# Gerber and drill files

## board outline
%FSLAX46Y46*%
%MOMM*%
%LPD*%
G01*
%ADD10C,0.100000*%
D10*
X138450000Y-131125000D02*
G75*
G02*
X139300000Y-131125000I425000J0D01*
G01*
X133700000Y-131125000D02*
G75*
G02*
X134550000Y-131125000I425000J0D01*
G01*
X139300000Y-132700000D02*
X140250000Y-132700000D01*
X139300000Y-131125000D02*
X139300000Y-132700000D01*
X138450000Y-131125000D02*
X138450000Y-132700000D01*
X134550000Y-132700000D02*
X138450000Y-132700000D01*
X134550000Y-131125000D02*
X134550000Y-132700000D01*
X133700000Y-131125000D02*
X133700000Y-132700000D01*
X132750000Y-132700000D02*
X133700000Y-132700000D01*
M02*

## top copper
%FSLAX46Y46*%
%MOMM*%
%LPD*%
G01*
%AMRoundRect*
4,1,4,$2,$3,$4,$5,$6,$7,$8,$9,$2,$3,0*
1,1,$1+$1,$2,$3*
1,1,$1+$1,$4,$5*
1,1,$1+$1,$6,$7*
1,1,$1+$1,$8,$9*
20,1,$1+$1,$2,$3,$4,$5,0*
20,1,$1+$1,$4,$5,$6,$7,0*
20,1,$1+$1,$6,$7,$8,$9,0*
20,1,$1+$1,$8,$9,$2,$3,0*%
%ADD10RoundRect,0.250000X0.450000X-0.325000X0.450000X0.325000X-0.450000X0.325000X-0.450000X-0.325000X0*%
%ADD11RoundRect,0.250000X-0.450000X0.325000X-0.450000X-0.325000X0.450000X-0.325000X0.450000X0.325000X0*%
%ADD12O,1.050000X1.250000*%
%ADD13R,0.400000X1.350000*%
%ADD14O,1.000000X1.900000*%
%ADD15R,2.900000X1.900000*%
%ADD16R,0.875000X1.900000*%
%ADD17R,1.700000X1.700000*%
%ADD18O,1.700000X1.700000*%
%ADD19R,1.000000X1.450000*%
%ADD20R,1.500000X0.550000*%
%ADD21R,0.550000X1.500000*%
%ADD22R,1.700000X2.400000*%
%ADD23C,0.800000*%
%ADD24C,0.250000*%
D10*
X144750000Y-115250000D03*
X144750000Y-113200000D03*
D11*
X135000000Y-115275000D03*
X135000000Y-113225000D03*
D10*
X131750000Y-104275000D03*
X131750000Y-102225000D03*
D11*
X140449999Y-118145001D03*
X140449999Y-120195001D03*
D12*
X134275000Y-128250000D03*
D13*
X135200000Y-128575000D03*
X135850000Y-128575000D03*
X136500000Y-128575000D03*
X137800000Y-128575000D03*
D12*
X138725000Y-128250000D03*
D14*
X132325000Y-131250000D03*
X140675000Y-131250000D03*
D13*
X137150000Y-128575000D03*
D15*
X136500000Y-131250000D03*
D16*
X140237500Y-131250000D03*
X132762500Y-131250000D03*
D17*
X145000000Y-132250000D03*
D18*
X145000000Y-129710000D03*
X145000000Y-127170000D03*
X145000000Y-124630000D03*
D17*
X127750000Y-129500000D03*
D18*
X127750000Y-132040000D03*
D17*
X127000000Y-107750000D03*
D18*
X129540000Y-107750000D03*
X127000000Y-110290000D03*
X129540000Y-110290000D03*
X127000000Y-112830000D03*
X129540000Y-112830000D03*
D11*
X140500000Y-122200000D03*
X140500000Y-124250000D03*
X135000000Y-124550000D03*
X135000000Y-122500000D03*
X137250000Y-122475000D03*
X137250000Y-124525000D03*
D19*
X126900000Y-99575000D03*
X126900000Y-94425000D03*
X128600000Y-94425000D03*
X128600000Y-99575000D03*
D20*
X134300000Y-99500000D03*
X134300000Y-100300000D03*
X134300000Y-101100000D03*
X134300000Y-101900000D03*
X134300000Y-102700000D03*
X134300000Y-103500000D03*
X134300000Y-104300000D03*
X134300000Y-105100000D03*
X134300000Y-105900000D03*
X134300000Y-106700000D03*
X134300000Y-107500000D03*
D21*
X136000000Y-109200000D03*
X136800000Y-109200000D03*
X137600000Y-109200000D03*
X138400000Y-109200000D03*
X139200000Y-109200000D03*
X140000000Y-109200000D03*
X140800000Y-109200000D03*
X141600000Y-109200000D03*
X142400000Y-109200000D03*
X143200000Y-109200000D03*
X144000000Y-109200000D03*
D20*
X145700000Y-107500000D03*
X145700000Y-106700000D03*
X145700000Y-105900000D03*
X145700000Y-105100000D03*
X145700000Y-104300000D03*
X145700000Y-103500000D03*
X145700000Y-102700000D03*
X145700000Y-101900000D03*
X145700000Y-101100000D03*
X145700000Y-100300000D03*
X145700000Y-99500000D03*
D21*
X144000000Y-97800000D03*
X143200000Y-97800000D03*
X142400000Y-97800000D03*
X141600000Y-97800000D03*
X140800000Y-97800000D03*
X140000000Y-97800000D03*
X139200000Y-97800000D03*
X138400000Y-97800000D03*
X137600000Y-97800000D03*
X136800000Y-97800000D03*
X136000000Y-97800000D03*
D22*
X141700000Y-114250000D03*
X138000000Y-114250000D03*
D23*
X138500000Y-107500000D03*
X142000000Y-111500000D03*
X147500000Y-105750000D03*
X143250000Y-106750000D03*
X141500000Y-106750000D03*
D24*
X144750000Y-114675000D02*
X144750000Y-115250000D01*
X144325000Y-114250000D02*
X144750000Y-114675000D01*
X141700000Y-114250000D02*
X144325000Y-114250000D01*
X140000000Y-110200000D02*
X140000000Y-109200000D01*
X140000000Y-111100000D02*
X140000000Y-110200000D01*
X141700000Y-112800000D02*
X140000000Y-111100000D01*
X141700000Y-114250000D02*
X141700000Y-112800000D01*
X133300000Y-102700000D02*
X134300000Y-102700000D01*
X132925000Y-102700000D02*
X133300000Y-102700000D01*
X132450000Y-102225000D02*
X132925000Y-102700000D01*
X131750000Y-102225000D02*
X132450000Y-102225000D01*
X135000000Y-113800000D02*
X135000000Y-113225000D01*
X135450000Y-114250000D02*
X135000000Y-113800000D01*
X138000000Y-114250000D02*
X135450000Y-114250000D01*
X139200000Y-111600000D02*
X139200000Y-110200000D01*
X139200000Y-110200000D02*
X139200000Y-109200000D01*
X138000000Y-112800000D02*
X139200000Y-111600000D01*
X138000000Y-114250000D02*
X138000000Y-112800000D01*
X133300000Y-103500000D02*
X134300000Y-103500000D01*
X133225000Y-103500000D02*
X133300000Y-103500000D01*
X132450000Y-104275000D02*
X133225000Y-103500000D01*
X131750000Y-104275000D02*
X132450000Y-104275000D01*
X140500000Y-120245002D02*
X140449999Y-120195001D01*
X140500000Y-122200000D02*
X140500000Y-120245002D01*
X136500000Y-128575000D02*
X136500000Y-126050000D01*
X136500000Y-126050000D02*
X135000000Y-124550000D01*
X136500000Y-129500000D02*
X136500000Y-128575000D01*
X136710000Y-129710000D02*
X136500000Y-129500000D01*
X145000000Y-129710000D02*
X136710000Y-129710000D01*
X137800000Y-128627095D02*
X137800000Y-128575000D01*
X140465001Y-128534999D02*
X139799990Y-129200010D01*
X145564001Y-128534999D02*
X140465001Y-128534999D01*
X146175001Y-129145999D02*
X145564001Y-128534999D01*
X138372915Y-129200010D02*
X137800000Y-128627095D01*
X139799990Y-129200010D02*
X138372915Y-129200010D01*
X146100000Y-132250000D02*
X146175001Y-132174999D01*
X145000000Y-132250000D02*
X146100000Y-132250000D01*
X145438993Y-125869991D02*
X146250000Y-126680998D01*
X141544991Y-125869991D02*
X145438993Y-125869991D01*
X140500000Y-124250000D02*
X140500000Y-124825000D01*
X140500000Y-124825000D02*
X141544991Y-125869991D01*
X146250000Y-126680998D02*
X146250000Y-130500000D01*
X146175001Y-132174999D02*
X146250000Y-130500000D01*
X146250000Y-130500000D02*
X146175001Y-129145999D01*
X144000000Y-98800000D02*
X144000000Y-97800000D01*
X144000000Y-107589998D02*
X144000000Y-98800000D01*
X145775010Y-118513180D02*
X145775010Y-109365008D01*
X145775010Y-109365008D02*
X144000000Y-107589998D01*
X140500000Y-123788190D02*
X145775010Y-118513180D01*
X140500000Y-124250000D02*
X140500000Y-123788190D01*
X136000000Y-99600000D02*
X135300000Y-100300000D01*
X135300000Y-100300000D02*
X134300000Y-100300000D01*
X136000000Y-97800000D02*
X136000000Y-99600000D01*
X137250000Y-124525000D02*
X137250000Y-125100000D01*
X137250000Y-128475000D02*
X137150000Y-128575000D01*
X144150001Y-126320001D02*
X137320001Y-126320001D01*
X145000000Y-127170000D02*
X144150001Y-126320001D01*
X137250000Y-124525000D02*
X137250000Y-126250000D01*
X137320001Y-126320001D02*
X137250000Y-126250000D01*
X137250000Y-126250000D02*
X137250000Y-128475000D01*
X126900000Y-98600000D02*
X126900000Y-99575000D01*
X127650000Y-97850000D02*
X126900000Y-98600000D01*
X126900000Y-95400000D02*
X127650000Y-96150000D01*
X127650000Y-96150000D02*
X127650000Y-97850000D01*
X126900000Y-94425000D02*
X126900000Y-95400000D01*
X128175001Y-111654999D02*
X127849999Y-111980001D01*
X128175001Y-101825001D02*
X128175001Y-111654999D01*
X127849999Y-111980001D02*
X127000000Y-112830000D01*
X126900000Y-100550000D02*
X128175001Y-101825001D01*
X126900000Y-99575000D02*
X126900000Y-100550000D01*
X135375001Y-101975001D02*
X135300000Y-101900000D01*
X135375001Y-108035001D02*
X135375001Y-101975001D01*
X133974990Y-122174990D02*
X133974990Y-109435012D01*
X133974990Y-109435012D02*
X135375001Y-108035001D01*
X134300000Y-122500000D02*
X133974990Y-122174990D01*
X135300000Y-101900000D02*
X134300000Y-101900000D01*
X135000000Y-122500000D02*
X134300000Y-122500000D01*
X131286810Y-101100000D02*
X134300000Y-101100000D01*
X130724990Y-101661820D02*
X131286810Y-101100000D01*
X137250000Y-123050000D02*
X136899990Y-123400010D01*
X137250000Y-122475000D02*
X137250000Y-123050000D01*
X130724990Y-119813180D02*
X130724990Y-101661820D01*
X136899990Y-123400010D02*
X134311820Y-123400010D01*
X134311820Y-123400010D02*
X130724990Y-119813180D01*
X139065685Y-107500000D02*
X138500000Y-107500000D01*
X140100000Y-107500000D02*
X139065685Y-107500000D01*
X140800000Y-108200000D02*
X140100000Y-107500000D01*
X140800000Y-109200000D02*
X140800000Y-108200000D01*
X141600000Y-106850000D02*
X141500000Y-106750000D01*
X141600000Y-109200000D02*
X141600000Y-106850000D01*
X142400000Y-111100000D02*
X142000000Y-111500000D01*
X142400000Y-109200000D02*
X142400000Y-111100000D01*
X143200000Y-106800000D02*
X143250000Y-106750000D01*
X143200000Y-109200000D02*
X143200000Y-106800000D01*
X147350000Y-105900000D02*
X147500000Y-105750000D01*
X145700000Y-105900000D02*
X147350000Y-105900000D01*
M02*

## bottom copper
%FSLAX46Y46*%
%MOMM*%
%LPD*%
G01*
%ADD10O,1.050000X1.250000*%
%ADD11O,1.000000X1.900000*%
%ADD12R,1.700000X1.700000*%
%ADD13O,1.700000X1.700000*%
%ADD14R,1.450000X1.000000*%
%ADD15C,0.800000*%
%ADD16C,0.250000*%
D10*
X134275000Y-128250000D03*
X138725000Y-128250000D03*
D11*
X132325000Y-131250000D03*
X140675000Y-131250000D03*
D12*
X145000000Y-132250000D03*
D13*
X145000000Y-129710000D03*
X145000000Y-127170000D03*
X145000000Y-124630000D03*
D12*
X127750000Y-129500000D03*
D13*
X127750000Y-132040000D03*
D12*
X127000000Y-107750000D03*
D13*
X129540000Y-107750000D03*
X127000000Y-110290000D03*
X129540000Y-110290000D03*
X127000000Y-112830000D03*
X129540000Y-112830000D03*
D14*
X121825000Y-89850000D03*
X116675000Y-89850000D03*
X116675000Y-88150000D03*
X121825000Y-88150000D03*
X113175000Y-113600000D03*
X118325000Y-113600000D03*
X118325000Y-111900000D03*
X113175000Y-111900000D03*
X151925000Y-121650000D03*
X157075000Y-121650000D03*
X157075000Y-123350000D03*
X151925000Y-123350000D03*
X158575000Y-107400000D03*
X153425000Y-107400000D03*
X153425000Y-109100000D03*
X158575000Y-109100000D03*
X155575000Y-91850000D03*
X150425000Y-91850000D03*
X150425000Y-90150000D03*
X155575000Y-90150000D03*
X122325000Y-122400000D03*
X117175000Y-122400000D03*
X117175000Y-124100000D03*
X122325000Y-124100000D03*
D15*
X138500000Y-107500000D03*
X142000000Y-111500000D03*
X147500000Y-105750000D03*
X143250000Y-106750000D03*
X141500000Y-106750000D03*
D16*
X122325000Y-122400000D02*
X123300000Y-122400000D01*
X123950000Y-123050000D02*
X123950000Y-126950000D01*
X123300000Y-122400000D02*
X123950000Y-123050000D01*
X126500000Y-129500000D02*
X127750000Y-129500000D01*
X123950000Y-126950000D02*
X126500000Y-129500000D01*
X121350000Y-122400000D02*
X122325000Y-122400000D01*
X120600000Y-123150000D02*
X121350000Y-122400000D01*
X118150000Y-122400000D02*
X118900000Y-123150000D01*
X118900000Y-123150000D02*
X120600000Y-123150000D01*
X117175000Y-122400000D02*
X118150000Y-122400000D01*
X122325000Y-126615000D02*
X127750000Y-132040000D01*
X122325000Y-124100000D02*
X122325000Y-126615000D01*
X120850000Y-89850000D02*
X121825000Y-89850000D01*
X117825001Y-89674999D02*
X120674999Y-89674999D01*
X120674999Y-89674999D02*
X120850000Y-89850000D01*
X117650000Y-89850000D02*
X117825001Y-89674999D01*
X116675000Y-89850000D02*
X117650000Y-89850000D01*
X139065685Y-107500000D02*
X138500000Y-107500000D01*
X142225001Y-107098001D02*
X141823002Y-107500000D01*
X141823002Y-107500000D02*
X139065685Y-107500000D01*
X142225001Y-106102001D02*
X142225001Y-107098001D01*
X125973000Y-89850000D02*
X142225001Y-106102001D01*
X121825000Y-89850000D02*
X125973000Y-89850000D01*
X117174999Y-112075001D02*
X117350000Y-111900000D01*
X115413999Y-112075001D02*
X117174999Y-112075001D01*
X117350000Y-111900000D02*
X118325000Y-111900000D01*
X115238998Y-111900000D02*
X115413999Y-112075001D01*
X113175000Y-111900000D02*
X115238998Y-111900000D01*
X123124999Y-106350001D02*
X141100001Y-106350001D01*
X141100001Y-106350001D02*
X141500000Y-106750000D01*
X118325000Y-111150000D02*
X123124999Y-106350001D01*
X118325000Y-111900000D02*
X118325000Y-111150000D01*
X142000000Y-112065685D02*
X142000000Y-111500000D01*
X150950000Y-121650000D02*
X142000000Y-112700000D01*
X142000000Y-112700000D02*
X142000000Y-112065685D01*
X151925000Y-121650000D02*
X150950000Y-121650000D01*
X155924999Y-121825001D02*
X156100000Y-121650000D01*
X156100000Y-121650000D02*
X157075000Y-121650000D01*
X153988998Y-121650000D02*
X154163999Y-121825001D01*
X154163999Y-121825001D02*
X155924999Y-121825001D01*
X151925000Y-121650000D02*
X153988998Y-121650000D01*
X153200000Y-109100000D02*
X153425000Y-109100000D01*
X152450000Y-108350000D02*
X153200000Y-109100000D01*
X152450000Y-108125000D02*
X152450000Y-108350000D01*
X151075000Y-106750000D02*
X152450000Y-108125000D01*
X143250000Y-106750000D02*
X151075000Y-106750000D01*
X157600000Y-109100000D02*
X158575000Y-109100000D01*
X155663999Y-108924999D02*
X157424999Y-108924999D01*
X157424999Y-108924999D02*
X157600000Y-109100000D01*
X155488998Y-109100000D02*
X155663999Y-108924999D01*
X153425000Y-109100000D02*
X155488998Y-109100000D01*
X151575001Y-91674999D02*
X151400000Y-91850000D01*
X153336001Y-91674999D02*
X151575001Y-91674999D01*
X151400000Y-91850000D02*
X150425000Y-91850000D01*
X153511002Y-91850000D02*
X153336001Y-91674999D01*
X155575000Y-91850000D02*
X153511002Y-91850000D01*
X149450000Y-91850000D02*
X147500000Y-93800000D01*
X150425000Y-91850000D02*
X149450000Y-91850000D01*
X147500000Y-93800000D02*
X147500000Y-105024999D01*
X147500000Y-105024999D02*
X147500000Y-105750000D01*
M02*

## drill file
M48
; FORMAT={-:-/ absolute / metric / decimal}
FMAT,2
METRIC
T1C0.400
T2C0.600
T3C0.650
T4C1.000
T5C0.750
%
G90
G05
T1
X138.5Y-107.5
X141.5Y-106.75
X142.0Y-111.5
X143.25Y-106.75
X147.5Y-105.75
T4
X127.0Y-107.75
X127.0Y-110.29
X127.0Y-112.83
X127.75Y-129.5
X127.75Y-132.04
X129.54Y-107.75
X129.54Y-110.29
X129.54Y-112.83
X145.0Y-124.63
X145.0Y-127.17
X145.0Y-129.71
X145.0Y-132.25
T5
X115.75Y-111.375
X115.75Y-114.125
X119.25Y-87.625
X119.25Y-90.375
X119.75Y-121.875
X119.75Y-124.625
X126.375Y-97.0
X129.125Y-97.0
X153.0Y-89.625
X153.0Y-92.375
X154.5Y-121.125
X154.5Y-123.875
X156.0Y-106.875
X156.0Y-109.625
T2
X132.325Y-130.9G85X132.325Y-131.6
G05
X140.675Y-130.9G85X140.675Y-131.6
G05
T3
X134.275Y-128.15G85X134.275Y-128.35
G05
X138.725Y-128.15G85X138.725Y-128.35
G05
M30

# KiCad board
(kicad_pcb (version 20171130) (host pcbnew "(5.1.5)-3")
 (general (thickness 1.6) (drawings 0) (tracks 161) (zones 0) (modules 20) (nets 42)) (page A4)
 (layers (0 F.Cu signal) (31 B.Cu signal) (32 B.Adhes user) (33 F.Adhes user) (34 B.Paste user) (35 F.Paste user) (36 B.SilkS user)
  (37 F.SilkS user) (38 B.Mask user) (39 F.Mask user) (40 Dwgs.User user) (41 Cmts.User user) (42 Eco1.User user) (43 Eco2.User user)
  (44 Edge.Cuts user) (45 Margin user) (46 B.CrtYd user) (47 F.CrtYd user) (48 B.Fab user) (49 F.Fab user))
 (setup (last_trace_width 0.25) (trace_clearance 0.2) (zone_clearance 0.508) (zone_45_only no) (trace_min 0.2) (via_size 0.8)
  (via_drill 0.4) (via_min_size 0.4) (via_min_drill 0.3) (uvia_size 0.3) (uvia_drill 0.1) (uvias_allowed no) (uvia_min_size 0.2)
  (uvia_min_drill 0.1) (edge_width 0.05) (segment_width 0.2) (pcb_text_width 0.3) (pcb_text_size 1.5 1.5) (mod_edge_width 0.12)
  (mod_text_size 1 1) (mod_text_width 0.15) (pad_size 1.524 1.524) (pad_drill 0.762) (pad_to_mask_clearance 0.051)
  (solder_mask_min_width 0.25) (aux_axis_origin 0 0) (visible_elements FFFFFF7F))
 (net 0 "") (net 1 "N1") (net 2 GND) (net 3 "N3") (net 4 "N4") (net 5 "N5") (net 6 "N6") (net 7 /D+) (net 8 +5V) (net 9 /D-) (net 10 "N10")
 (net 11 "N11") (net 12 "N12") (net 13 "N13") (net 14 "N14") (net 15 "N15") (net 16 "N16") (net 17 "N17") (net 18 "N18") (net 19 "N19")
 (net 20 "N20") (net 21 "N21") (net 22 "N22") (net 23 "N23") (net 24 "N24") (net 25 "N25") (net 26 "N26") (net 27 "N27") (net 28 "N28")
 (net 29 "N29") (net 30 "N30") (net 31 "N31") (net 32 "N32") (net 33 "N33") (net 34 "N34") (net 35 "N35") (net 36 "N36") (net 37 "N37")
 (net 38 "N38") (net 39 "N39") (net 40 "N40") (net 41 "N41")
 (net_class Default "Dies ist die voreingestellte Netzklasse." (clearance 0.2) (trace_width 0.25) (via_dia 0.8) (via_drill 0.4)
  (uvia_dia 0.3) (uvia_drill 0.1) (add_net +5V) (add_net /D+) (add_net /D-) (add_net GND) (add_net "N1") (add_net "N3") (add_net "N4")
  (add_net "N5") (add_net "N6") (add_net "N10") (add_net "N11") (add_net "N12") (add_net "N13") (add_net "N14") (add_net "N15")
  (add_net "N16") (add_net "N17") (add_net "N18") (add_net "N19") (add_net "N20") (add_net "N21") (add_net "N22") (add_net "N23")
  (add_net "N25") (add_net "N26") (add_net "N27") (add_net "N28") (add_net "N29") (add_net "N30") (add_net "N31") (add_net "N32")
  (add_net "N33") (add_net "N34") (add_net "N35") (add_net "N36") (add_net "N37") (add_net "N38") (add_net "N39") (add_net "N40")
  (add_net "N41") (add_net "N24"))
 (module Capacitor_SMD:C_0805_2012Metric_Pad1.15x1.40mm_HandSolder (layer F.Cu) (at 144.75 114.225 90)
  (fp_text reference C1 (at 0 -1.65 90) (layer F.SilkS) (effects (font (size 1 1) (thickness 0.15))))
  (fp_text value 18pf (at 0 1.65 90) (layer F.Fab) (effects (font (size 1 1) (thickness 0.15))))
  (pad 1 smd roundrect (at -1.025 0 90) (size 1.15 1.4) (layers F.Cu F.Paste F.Mask) (roundrect_rratio 0.217391) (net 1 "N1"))
  (pad 2 smd roundrect (at 1.025 0 90) (size 1.15 1.4) (layers F.Cu F.Paste F.Mask) (roundrect_rratio 0.217391) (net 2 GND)))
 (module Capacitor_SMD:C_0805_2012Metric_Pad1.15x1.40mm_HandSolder (layer F.Cu) (at 135 114.25 270)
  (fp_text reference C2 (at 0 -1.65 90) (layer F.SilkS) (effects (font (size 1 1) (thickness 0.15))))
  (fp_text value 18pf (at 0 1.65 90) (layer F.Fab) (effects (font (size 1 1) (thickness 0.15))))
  (pad 2 smd roundrect (at 1.025 0 270) (size 1.15 1.4) (layers F.Cu F.Paste F.Mask) (roundrect_rratio 0.217391) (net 2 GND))
  (pad 1 smd roundrect (at -1.025 0 270) (size 1.15 1.4) (layers F.Cu F.Paste F.Mask) (roundrect_rratio 0.217391) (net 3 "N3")))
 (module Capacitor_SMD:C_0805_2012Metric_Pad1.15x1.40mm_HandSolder (layer F.Cu) (at 131.75 103.25 90)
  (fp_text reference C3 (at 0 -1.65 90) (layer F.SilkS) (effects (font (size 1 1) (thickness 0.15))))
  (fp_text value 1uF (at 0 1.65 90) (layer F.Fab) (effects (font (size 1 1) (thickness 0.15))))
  (pad 1 smd roundrect (at -1.025 0 90) (size 1.15 1.4) (layers F.Cu F.Paste F.Mask) (roundrect_rratio 0.217391) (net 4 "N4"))
  (pad 2 smd roundrect (at 1.025 0 90) (size 1.15 1.4) (layers F.Cu F.Paste F.Mask) (roundrect_rratio 0.217391) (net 2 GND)))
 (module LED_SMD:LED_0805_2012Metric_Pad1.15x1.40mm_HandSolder (layer F.Cu) (at 140.449999 119.170001 270)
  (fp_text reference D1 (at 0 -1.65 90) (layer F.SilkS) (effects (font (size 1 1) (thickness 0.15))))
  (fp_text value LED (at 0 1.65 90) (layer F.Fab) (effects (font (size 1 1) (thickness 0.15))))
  (pad 1 smd roundrect (at -1.025 0 270) (size 1.15 1.4) (layers F.Cu F.Paste F.Mask) (roundrect_rratio 0.217391) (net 2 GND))
  (pad 2 smd roundrect (at 1.025 0 270) (size 1.15 1.4) (layers F.Cu F.Paste F.Mask) (roundrect_rratio 0.217391) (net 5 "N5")))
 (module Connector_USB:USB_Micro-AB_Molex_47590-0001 (layer F.Cu) (at 136.5 131.25)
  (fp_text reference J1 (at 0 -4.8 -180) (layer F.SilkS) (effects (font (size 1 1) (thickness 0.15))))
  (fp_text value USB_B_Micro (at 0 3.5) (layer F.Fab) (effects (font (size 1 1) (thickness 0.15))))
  (fp_arc (start 2.375 -0.125) (end 1.95 -0.125) (angle 180) (layer Edge.Cuts) (width 0.1))
  (fp_arc (start -2.375 -0.125) (end -2.8 -0.125) (angle 180) (layer Edge.Cuts) (width 0.1))
  (fp_line (start 2.8 1.45) (end 3.75 1.45) (layer Edge.Cuts) (width 0.1))
  (fp_line (start 2.8 -0.125) (end 2.8 1.45) (layer Edge.Cuts) (width 0.1))
  (fp_line (start 1.95 -0.125) (end 1.95 1.45) (layer Edge.Cuts) (width 0.1))
  (fp_line (start -1.95 1.45) (end 1.95 1.45) (layer Edge.Cuts) (width 0.1))
  (fp_line (start -1.95 -0.125) (end -1.95 1.45) (layer Edge.Cuts) (width 0.1))
  (fp_line (start -2.8 -0.125) (end -2.8 1.45) (layer Edge.Cuts) (width 0.1))
  (fp_line (start -3.75 1.45) (end -2.8 1.45) (layer Edge.Cuts) (width 0.1))
  (pad 6 thru_hole oval (at -2.225 -3) (size 1.05 1.25) (drill oval 0.65 0.85) (layers *.Cu *.Mask) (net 2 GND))
  (pad 5 smd rect (at -1.3 -2.675) (size 0.4 1.35) (layers F.Cu F.Paste F.Mask) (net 2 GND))
  (pad 4 smd rect (at -0.65 -2.675) (size 0.4 1.35) (layers F.Cu F.Paste F.Mask) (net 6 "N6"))
  (pad 3 smd rect (at 0 -2.675) (size 0.4 1.35) (layers F.Cu F.Paste F.Mask) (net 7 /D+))
  (pad 1 smd rect (at 1.3 -2.675) (size 0.4 1.35) (layers F.Cu F.Paste F.Mask) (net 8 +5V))
  (pad 6 thru_hole oval (at 2.225 -3) (size 1.05 1.25) (drill oval 0.65 0.85) (layers *.Cu *.Mask) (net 2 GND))
  (pad 6 thru_hole oval (at -4.175 0) (size 1 1.9) (drill oval 0.6 1.3) (layers *.Cu *.Mask) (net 2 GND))
  (pad 6 thru_hole oval (at 4.175 0) (size 1 1.9) (drill oval 0.6 1.3) (layers *.Cu *.Mask) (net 2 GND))
  (pad 2 smd rect (at 0.65 -2.675) (size 0.4 1.35) (layers F.Cu F.Paste F.Mask) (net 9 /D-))
  (pad 6 smd rect (at 0 0) (size 2.9 1.9) (layers F.Cu F.Paste F.Mask) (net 2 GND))
  (pad 6 smd rect (at 3.7375 0) (size 0.875 1.9) (layers F.Cu F.Mask) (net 2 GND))
  (pad 6 smd rect (at -3.7375 0) (size 0.875 1.9) (layers F.Cu F.Mask) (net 2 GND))
  (pad "" smd rect (at 3.5 0) (size 0.3 0.85) (layers F.Paste))
  (pad "" smd rect (at -3.5 0) (size 0.3 0.85) (layers F.Paste)))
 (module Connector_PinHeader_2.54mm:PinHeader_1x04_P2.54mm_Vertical (layer F.Cu) (at 145 132.25 180)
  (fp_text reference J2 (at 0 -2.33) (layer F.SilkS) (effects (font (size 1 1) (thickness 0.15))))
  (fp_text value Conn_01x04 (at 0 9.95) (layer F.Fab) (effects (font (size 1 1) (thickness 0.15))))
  (pad 1 thru_hole rect (at 0 0 180) (size 1.7 1.7) (drill 1) (layers *.Cu *.Mask) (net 8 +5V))
  (pad 2 thru_hole oval (at 0 2.54 180) (size 1.7 1.7) (drill 1) (layers *.Cu *.Mask) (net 7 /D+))
  (pad 3 thru_hole oval (at 0 5.08 180) (size 1.7 1.7) (drill 1) (layers *.Cu *.Mask) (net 9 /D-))
  (pad 4 thru_hole oval (at 0 7.62 180) (size 1.7 1.7) (drill 1) (layers *.Cu *.Mask) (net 2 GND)))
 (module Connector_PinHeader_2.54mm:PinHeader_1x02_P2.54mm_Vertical (layer F.Cu) (at 127.75 129.5)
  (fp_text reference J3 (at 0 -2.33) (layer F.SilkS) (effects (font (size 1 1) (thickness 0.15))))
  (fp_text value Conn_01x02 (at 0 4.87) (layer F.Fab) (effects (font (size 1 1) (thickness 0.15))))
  (pad 1 thru_hole rect (at 0 0) (size 1.7 1.7) (drill 1) (layers *.Cu *.Mask) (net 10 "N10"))
  (pad 2 thru_hole oval (at 0 2.54) (size 1.7 1.7) (drill 1) (layers *.Cu *.Mask) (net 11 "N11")))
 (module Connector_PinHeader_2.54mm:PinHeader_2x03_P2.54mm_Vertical (layer F.Cu) (at 127 107.75)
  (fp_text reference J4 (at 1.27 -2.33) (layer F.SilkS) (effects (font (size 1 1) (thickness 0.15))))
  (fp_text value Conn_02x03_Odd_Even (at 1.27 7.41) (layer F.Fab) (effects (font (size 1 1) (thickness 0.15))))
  (pad 1 thru_hole rect (at 0 0) (size 1.7 1.7) (drill 1) (layers *.Cu *.Mask) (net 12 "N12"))
  (pad 2 thru_hole oval (at 2.54 0) (size 1.7 1.7) (drill 1) (layers *.Cu *.Mask) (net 8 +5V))
  (pad 3 thru_hole oval (at 0 2.54) (size 1.7 1.7) (drill 1) (layers *.Cu *.Mask) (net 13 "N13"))
  (pad 4 thru_hole oval (at 2.54 2.54) (size 1.7 1.7) (drill 1) (layers *.Cu *.Mask) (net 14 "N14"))
  (pad 5 thru_hole oval (at 0 5.08) (size 1.7 1.7) (drill 1) (layers *.Cu *.Mask) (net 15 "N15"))
  (pad 6 thru_hole oval (at 2.54 5.08) (size 1.7 1.7) (drill 1) (layers *.Cu *.Mask) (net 2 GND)))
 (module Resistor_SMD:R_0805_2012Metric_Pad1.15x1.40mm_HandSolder (layer F.Cu) (at 140.5 123.225 270)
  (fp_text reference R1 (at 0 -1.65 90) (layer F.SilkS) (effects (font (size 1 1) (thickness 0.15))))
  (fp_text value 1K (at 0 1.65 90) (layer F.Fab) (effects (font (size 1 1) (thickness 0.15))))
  (pad 1 smd roundrect (at -1.025 0 270) (size 1.15 1.4) (layers F.Cu F.Paste F.Mask) (roundrect_rratio 0.217391) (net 5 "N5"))
  (pad 2 smd roundrect (at 1.025 0 270) (size 1.15 1.4) (layers F.Cu F.Paste F.Mask) (roundrect_rratio 0.217391) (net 8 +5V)))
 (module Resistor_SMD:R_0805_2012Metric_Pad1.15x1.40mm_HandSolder (layer F.Cu) (at 135 123.525 270)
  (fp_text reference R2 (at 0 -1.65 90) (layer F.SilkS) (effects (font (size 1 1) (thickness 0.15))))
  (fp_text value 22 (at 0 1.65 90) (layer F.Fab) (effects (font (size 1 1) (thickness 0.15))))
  (pad 2 smd roundrect (at 1.025 0 270) (size 1.15 1.4) (layers F.Cu F.Paste F.Mask) (roundrect_rratio 0.217391) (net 7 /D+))
  (pad 1 smd roundrect (at -1.025 0 270) (size 1.15 1.4) (layers F.Cu F.Paste F.Mask) (roundrect_rratio 0.217391) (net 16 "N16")))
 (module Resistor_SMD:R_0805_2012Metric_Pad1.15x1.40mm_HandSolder (layer F.Cu) (at 137.25 123.5 270)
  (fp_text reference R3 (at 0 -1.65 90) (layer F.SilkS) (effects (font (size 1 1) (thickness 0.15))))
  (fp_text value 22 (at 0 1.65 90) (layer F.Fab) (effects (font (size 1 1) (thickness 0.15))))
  (pad 1 smd roundrect (at -1.025 0 270) (size 1.15 1.4) (layers F.Cu F.Paste F.Mask) (roundrect_rratio 0.217391) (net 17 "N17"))
  (pad 2 smd roundrect (at 1.025 0 270) (size 1.15 1.4) (layers F.Cu F.Paste F.Mask) (roundrect_rratio 0.217391) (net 9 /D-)))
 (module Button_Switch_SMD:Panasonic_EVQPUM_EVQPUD (layer F.Cu) (at 127.75 97 270)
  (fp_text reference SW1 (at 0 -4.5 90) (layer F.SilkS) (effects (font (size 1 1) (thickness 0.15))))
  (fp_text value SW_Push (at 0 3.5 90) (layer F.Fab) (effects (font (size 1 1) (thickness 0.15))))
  (pad 2 smd rect (at 2.575 0.85 90) (size 1.45 1) (layers F.Cu F.Paste F.Mask) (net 15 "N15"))
  (pad 2 smd rect (at -2.575 0.85 90) (size 1.45 1) (layers F.Cu F.Paste F.Mask) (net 15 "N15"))
  (pad 1 smd rect (at -2.575 -0.85 90) (size 1.45 1) (layers F.Cu F.Paste F.Mask) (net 2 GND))
  (pad 1 smd rect (at 2.575 -0.85 90) (size 1.45 1) (layers F.Cu F.Paste F.Mask) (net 2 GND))
  (pad "" np_thru_hole circle (at 0 1.375 90) (size 0.75 0.75) (drill 0.75) (layers *.Cu *.Mask))
  (pad "" np_thru_hole circle (at 0 -1.375 90) (size 0.75 0.75) (drill 0.75) (layers *.Cu *.Mask)))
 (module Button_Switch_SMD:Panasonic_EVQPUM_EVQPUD (layer B.Cu) (at 119.25 89)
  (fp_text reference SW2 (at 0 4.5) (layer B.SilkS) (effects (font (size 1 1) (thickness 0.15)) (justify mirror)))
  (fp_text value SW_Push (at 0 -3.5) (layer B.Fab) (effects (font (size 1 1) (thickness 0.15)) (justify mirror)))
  (pad "" np_thru_hole circle (at 0 1.375 180) (size 0.75 0.75) (drill 0.75) (layers *.Cu *.Mask))
  (pad "" np_thru_hole circle (at 0 -1.375 180) (size 0.75 0.75) (drill 0.75) (layers *.Cu *.Mask))
  (pad 1 smd rect (at 2.575 0.85 180) (size 1.45 1) (layers B.Cu B.Paste B.Mask) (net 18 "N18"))
  (pad 1 smd rect (at -2.575 0.85 180) (size 1.45 1) (layers B.Cu B.Paste B.Mask) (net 18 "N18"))
  (pad 2 smd rect (at -2.575 -0.85 180) (size 1.45 1) (layers B.Cu B.Paste B.Mask) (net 2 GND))
  (pad 2 smd rect (at 2.575 -0.85 180) (size 1.45 1) (layers B.Cu B.Paste B.Mask) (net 2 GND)))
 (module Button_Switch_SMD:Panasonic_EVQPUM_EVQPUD (layer B.Cu) (at 115.75 112.75 180)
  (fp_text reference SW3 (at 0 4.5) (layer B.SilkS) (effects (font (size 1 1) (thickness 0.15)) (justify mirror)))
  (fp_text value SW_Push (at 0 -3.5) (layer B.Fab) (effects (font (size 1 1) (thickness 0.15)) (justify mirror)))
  (pad 2 smd rect (at 2.575 -0.85) (size 1.45 1) (layers B.Cu B.Paste B.Mask) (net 2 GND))
  (pad 2 smd rect (at -2.575 -0.85) (size 1.45 1) (layers B.Cu B.Paste B.Mask) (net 2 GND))
  (pad 1 smd rect (at -2.575 0.85) (size 1.45 1) (layers B.Cu B.Paste B.Mask) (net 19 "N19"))
  (pad 1 smd rect (at 2.575 0.85) (size 1.45 1) (layers B.Cu B.Paste B.Mask) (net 19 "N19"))
  (pad "" np_thru_hole circle (at 0 -1.375) (size 0.75 0.75) (drill 0.75) (layers *.Cu *.Mask))
  (pad "" np_thru_hole circle (at 0 1.375) (size 0.75 0.75) (drill 0.75) (layers *.Cu *.Mask)))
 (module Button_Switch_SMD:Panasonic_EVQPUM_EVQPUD (layer B.Cu) (at 154.5 122.5 180)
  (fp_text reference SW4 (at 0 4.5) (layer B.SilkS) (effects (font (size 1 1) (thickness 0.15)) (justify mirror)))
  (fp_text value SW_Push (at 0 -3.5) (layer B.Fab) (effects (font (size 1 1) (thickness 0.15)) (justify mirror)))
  (pad "" np_thru_hole circle (at 0 1.375) (size 0.75 0.75) (drill 0.75) (layers *.Cu *.Mask))
  (pad "" np_thru_hole circle (at 0 -1.375) (size 0.75 0.75) (drill 0.75) (layers *.Cu *.Mask))
  (pad 1 smd rect (at 2.575 0.85) (size 1.45 1) (layers B.Cu B.Paste B.Mask) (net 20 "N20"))
  (pad 1 smd rect (at -2.575 0.85) (size 1.45 1) (layers B.Cu B.Paste B.Mask) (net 20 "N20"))
  (pad 2 smd rect (at -2.575 -0.85) (size 1.45 1) (layers B.Cu B.Paste B.Mask) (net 2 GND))
  (pad 2 smd rect (at 2.575 -0.85) (size 1.45 1) (layers B.Cu B.Paste B.Mask) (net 2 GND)))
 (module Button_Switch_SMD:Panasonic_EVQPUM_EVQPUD (layer B.Cu) (at 156 108.25)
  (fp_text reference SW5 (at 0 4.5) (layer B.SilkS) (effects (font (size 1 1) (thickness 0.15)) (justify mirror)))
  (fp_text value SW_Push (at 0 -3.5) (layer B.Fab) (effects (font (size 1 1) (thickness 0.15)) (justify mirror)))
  (pad 2 smd rect (at 2.575 -0.85 180) (size 1.45 1) (layers B.Cu B.Paste B.Mask) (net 2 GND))
  (pad 2 smd rect (at -2.575 -0.85 180) (size 1.45 1) (layers B.Cu B.Paste B.Mask) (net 2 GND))
  (pad 1 smd rect (at -2.575 0.85 180) (size 1.45 1) (layers B.Cu B.Paste B.Mask) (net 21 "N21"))
  (pad 1 smd rect (at 2.575 0.85 180) (size 1.45 1) (layers B.Cu B.Paste B.Mask) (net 21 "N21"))
  (pad "" np_thru_hole circle (at 0 -1.375 180) (size 0.75 0.75) (drill 0.75) (layers *.Cu *.Mask))
  (pad "" np_thru_hole circle (at 0 1.375 180) (size 0.75 0.75) (drill 0.75) (layers *.Cu *.Mask)))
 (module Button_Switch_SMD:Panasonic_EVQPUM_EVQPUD (layer B.Cu) (at 153 91)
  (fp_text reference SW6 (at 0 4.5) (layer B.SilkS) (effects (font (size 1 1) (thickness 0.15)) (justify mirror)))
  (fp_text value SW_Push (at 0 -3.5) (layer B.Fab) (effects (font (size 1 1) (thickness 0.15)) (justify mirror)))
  (pad "" np_thru_hole circle (at 0 1.375 180) (size 0.75 0.75) (drill 0.75) (layers *.Cu *.Mask))
  (pad "" np_thru_hole circle (at 0 -1.375 180) (size 0.75 0.75) (drill 0.75) (layers *.Cu *.Mask))
  (pad 1 smd rect (at 2.575 0.85 180) (size 1.45 1) (layers B.Cu B.Paste B.Mask) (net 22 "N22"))
  (pad 1 smd rect (at -2.575 0.85 180) (size 1.45 1) (layers B.Cu B.Paste B.Mask) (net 22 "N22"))
  (pad 2 smd rect (at -2.575 -0.85 180) (size 1.45 1) (layers B.Cu B.Paste B.Mask) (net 2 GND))
  (pad 2 smd rect (at 2.575 -0.85 180) (size 1.45 1) (layers B.Cu B.Paste B.Mask) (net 2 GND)))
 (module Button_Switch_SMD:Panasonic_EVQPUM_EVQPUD (layer B.Cu) (at 119.75 123.25)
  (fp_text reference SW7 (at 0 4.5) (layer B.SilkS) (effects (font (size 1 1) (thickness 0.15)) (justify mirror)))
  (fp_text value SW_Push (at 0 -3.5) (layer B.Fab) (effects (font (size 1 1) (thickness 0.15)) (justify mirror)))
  (pad 2 smd rect (at 2.575 -0.85 180) (size 1.45 1) (layers B.Cu B.Paste B.Mask) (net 10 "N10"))
  (pad 2 smd rect (at -2.575 -0.85 180) (size 1.45 1) (layers B.Cu B.Paste B.Mask) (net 10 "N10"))
  (pad 1 smd rect (at -2.575 0.85 180) (size 1.45 1) (layers B.Cu B.Paste B.Mask) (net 11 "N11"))
  (pad 1 smd rect (at 2.575 0.85 180) (size 1.45 1) (layers B.Cu B.Paste B.Mask) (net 11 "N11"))
  (pad "" np_thru_hole circle (at 0 -1.375 180) (size 0.75 0.75) (drill 0.75) (layers *.Cu *.Mask))
  (pad "" np_thru_hole circle (at 0 1.375 180) (size 0.75 0.75) (drill 0.75) (layers *.Cu *.Mask)))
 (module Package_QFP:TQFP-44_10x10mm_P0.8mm (layer F.Cu) (at 140 103.5)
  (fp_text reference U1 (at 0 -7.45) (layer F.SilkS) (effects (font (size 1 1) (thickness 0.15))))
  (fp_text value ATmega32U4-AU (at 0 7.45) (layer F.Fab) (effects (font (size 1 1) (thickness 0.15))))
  (pad 1 smd rect (at -5.7 -4) (size 1.5 0.55) (layers F.Cu F.Paste F.Mask) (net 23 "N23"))
  (pad 2 smd rect (at -5.7 -3.2) (size 1.5 0.55) (layers F.Cu F.Paste F.Mask) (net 8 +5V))
  (pad 3 smd rect (at -5.7 -2.4) (size 1.5 0.55) (layers F.Cu F.Paste F.Mask) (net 17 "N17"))
  (pad 4 smd rect (at -5.7 -1.6) (size 1.5 0.55) (layers F.Cu F.Paste F.Mask) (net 16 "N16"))
  (pad 5 smd rect (at -5.7 -0.8) (size 1.5 0.55) (layers F.Cu F.Paste F.Mask) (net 2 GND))
  (pad 6 smd rect (at -5.7 0) (size 1.5 0.55) (layers F.Cu F.Paste F.Mask) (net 4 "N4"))
  (pad 7 smd rect (at -5.7 0.8) (size 1.5 0.55) (layers F.Cu F.Paste F.Mask) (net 8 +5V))
  (pad 8 smd rect (at -5.7 1.6) (size 1.5 0.55) (layers F.Cu F.Paste F.Mask) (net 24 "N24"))
  (pad 9 smd rect (at -5.7 2.4) (size 1.5 0.55) (layers F.Cu F.Paste F.Mask) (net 13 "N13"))
  (pad 10 smd rect (at -5.7 3.2) (size 1.5 0.55) (layers F.Cu F.Paste F.Mask) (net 14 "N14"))
  (pad 11 smd rect (at -5.7 4) (size 1.5 0.55) (layers F.Cu F.Paste F.Mask) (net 12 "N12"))
  (pad 12 smd rect (at -4 5.7 90) (size 1.5 0.55) (layers F.Cu F.Paste F.Mask) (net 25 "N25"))
  (pad 13 smd rect (at -3.2 5.7 90) (size 1.5 0.55) (layers F.Cu F.Paste F.Mask) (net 15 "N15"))
  (pad 14 smd rect (at -2.4 5.7 90) (size 1.5 0.55) (layers F.Cu F.Paste F.Mask) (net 8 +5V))
  (pad 15 smd rect (at -1.6 5.7 90) (size 1.5 0.55) (layers F.Cu F.Paste F.Mask) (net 2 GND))
  (pad 16 smd rect (at -0.8 5.7 90) (size 1.5 0.55) (layers F.Cu F.Paste F.Mask) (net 3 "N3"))
  (pad 17 smd rect (at 0 5.7 90) (size 1.5 0.55) (layers F.Cu F.Paste F.Mask) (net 1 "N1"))
  (pad 18 smd rect (at 0.8 5.7 90) (size 1.5 0.55) (layers F.Cu F.Paste F.Mask) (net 18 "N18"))
  (pad 19 smd rect (at 1.6 5.7 90) (size 1.5 0.55) (layers F.Cu F.Paste F.Mask) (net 19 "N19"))
  (pad 20 smd rect (at 2.4 5.7 90) (size 1.5 0.55) (layers F.Cu F.Paste F.Mask) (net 20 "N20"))
  (pad 21 smd rect (at 3.2 5.7 90) (size 1.5 0.55) (layers F.Cu F.Paste F.Mask) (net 21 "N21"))
  (pad 22 smd rect (at 4 5.7 90) (size 1.5 0.55) (layers F.Cu F.Paste F.Mask) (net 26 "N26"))
  (pad 23 smd rect (at 5.7 4) (size 1.5 0.55) (layers F.Cu F.Paste F.Mask) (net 2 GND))
  (pad 24 smd rect (at 5.7 3.2) (size 1.5 0.55) (layers F.Cu F.Paste F.Mask) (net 8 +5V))
  (pad 25 smd rect (at 5.7 2.4) (size 1.5 0.55) (layers F.Cu F.Paste F.Mask) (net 22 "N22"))
  (pad 26 smd rect (at 5.7 1.6) (size 1.5 0.55) (layers F.Cu F.Paste F.Mask) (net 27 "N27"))
  (pad 27 smd rect (at 5.7 0.8) (size 1.5 0.55) (layers F.Cu F.Paste F.Mask) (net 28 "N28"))
  (pad 28 smd rect (at 5.7 0) (size 1.5 0.55) (layers F.Cu F.Paste F.Mask) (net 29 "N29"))
  (pad 29 smd rect (at 5.7 -0.8) (size 1.5 0.55) (layers F.Cu F.Paste F.Mask) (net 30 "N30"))
  (pad 30 smd rect (at 5.7 -1.6) (size 1.5 0.55) (layers F.Cu F.Paste F.Mask) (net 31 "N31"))
  (pad 31 smd rect (at 5.7 -2.4) (size 1.5 0.55) (layers F.Cu F.Paste F.Mask) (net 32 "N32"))
  (pad 32 smd rect (at 5.7 -3.2) (size 1.5 0.55) (layers F.Cu F.Paste F.Mask) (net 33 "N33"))
  (pad 33 smd rect (at 5.7 -4) (size 1.5 0.55) (layers F.Cu F.Paste F.Mask) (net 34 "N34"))
  (pad 34 smd rect (at 4 -5.7 90) (size 1.5 0.55) (layers F.Cu F.Paste F.Mask) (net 8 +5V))
  (pad 35 smd rect (at 3.2 -5.7 90) (size 1.5 0.55) (layers F.Cu F.Paste F.Mask) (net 2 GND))
  (pad 36 smd rect (at 2.4 -5.7 90) (size 1.5 0.55) (layers F.Cu F.Paste F.Mask) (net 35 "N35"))
  (pad 37 smd rect (at 1.6 -5.7 90) (size 1.5 0.55) (layers F.Cu F.Paste F.Mask) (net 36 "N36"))
  (pad 38 smd rect (at 0.8 -5.7 90) (size 1.5 0.55) (layers F.Cu F.Paste F.Mask) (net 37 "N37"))
  (pad 39 smd rect (at 0 -5.7 90) (size 1.5 0.55) (layers F.Cu F.Paste F.Mask) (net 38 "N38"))
  (pad 40 smd rect (at -0.8 -5.7 90) (size 1.5 0.55) (layers F.Cu F.Paste F.Mask) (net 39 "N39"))
  (pad 41 smd rect (at -1.6 -5.7 90) (size 1.5 0.55) (layers F.Cu F.Paste F.Mask) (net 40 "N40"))
  (pad 42 smd rect (at -2.4 -5.7 90) (size 1.5 0.55) (layers F.Cu F.Paste F.Mask) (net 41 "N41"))
  (pad 43 smd rect (at -3.2 -5.7 90) (size 1.5 0.55) (layers F.Cu F.Paste F.Mask) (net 2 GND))
  (pad 44 smd rect (at -4 -5.7 90) (size 1.5 0.55) (layers F.Cu F.Paste F.Mask) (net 8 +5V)))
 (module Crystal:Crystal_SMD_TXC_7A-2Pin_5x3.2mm (layer F.Cu) (at 139.85 114.25 180)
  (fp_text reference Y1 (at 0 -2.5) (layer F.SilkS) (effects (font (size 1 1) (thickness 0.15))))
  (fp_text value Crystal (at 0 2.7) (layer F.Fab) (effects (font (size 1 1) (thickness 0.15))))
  (pad 1 smd rect (at -1.85 0 180) (size 1.7 2.4) (layers F.Cu F.Paste F.Mask) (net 1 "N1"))
  (pad 2 smd rect (at 1.85 0 180) (size 1.7 2.4) (layers F.Cu F.Paste F.Mask) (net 3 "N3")))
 (via (at 138.5 107.5) (size 0.8) (drill 0.4) (layers F.Cu B.Cu) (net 18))
 (via (at 142 111.5) (size 0.8) (drill 0.4) (layers F.Cu B.Cu) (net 20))
 (via (at 147.5 105.75) (size 0.8) (drill 0.4) (layers F.Cu B.Cu) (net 22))
 (via (at 143.25 106.75) (size 0.8) (drill 0.4) (layers F.Cu B.Cu) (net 21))
 (via (at 141.5 106.75) (size 0.8) (drill 0.4) (layers F.Cu B.Cu) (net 19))
 (segment (start 144.75 114.675) (end 144.75 115.25) (width 0.25) (layer F.Cu) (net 1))
 (segment (start 144.325 114.25) (end 144.75 114.675) (width 0.25) (layer F.Cu) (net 1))
 (segment (start 141.7 114.25) (end 144.325 114.25) (width 0.25) (layer F.Cu) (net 1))
 (segment (start 140 110.2) (end 140 109.2) (width 0.25) (layer F.Cu) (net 1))
 (segment (start 140 111.1) (end 140 110.2) (width 0.25) (layer F.Cu) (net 1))
 (segment (start 141.7 112.8) (end 140 111.1) (width 0.25) (layer F.Cu) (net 1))
 (segment (start 141.7 114.25) (end 141.7 112.8) (width 0.25) (layer F.Cu) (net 1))
 (segment (start 133.3 102.7) (end 134.3 102.7) (width 0.25) (layer F.Cu) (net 2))
 (segment (start 132.925 102.7) (end 133.3 102.7) (width 0.25) (layer F.Cu) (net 2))
 (segment (start 132.45 102.225) (end 132.925 102.7) (width 0.25) (layer F.Cu) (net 2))
 (segment (start 131.75 102.225) (end 132.45 102.225) (width 0.25) (layer F.Cu) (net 2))
 (segment (start 135 113.8) (end 135 113.225) (width 0.25) (layer F.Cu) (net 3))
 (segment (start 135.45 114.25) (end 135 113.8) (width 0.25) (layer F.Cu) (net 3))
 (segment (start 138 114.25) (end 135.45 114.25) (width 0.25) (layer F.Cu) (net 3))
 (segment (start 139.2 111.6) (end 139.2 110.2) (width 0.25) (layer F.Cu) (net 3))
 (segment (start 139.2 110.2) (end 139.2 109.2) (width 0.25) (layer F.Cu) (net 3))
 (segment (start 138 112.8) (end 139.2 111.6) (width 0.25) (layer F.Cu) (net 3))
 (segment (start 138 114.25) (end 138 112.8) (width 0.25) (layer F.Cu) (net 3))
 (segment (start 133.3 103.5) (end 134.3 103.5) (width 0.25) (layer F.Cu) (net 4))
 (segment (start 133.225 103.5) (end 133.3 103.5) (width 0.25) (layer F.Cu) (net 4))
 (segment (start 132.45 104.275) (end 133.225 103.5) (width 0.25) (layer F.Cu) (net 4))
 (segment (start 131.75 104.275) (end 132.45 104.275) (width 0.25) (layer F.Cu) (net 4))
 (segment (start 140.5 120.245002) (end 140.449999 120.195001) (width 0.25) (layer F.Cu) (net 5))
 (segment (start 140.5 122.2) (end 140.5 120.245002) (width 0.25) (layer F.Cu) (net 5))
 (segment (start 136.5 128.575) (end 136.5 126.05) (width 0.25) (layer F.Cu) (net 7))
 (segment (start 136.5 126.05) (end 135 124.55) (width 0.25) (layer F.Cu) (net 7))
 (segment (start 136.5 129.5) (end 136.5 128.575) (width 0.25) (layer F.Cu) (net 7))
 (segment (start 136.71 129.71) (end 136.5 129.5) (width 0.25) (layer F.Cu) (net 7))
 (segment (start 145 129.71) (end 136.71 129.71) (width 0.25) (layer F.Cu) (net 7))
 (segment (start 137.8 128.627095) (end 137.8 128.575) (width 0.25) (layer F.Cu) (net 8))
 (segment (start 140.465001 128.534999) (end 139.79999 129.20001) (width 0.25) (layer F.Cu) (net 8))
 (segment (start 145.564001 128.534999) (end 140.465001 128.534999) (width 0.25) (layer F.Cu) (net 8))
 (segment (start 146.175001 129.145999) (end 145.564001 128.534999) (width 0.25) (layer F.Cu) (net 8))
 (segment (start 138.372915 129.20001) (end 137.8 128.627095) (width 0.25) (layer F.Cu) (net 8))
 (segment (start 139.79999 129.20001) (end 138.372915 129.20001) (width 0.25) (layer F.Cu) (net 8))
 (segment (start 146.1 132.25) (end 146.175001 132.174999) (width 0.25) (layer F.Cu) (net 8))
 (segment (start 145 132.25) (end 146.1 132.25) (width 0.25) (layer F.Cu) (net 8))
 (segment (start 145.438993 125.869991) (end 146.25 126.680998) (width 0.25) (layer F.Cu) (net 8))
 (segment (start 141.544991 125.869991) (end 145.438993 125.869991) (width 0.25) (layer F.Cu) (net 8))
 (segment (start 140.5 124.25) (end 140.5 124.825) (width 0.25) (layer F.Cu) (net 8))
 (segment (start 140.5 124.825) (end 141.544991 125.869991) (width 0.25) (layer F.Cu) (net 8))
 (segment (start 146.25 126.680998) (end 146.25 130.5) (width 0.25) (layer F.Cu) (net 8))
 (segment (start 146.175001 132.174999) (end 146.25 130.5) (width 0.25) (layer F.Cu) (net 8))
 (segment (start 146.25 130.5) (end 146.175001 129.145999) (width 0.25) (layer F.Cu) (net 8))
 (segment (start 144 98.8) (end 144 97.8) (width 0.25) (layer F.Cu) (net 8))
 (segment (start 144 107.589998) (end 144 98.8) (width 0.25) (layer F.Cu) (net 8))
 (segment (start 145.77501 118.51318) (end 145.77501 109.365008) (width 0.25) (layer F.Cu) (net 8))
 (segment (start 145.77501 109.365008) (end 144 107.589998) (width 0.25) (layer F.Cu) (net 8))
 (segment (start 140.5 123.78819) (end 145.77501 118.51318) (width 0.25) (layer F.Cu) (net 8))
 (segment (start 140.5 124.25) (end 140.5 123.78819) (width 0.25) (layer F.Cu) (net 8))
 (segment (start 136 99.6) (end 135.3 100.3) (width 0.25) (layer F.Cu) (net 8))
 (segment (start 135.3 100.3) (end 134.3 100.3) (width 0.25) (layer F.Cu) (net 8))
 (segment (start 136 97.8) (end 136 99.6) (width 0.25) (layer F.Cu) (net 8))
 (segment (start 137.25 124.525) (end 137.25 125.1) (width 0.25) (layer F.Cu) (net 9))
 (segment (start 137.25 128.475) (end 137.15 128.575) (width 0.25) (layer F.Cu) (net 9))
 (segment (start 144.150001 126.320001) (end 137.320001 126.320001) (width 0.25) (layer F.Cu) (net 9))
 (segment (start 145 127.17) (end 144.150001 126.320001) (width 0.25) (layer F.Cu) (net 9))
 (segment (start 137.25 124.525) (end 137.25 126.25) (width 0.25) (layer F.Cu) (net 9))
 (segment (start 137.320001 126.320001) (end 137.25 126.25) (width 0.25) (layer F.Cu) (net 9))
 (segment (start 137.25 126.25) (end 137.25 128.475) (width 0.25) (layer F.Cu) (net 9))
 (segment (start 122.325 122.4) (end 123.3 122.4) (width 0.25) (layer B.Cu) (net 10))
 (segment (start 123.95 123.05) (end 123.95 126.95) (width 0.25) (layer B.Cu) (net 10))
 (segment (start 123.3 122.4) (end 123.95 123.05) (width 0.25) (layer B.Cu) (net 10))
 (segment (start 126.5 129.5) (end 127.75 129.5) (width 0.25) (layer B.Cu) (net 10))
 (segment (start 123.95 126.95) (end 126.5 129.5) (width 0.25) (layer B.Cu) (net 10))
 (segment (start 121.35 122.4) (end 122.325 122.4) (width 0.25) (layer B.Cu) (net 10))
 (segment (start 120.6 123.15) (end 121.35 122.4) (width 0.25) (layer B.Cu) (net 10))
 (segment (start 118.15 122.4) (end 118.9 123.15) (width 0.25) (layer B.Cu) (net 10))
 (segment (start 118.9 123.15) (end 120.6 123.15) (width 0.25) (layer B.Cu) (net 10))
 (segment (start 117.175 122.4) (end 118.15 122.4) (width 0.25) (layer B.Cu) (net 10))
 (segment (start 122.325 126.615) (end 127.75 132.04) (width 0.25) (layer B.Cu) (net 11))
 (segment (start 122.325 124.1) (end 122.325 126.615) (width 0.25) (layer B.Cu) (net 11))
 (segment (start 126.9 98.6) (end 126.9 99.575) (width 0.25) (layer F.Cu) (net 15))
 (segment (start 127.65 97.85) (end 126.9 98.6) (width 0.25) (layer F.Cu) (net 15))
 (segment (start 126.9 95.4) (end 127.65 96.15) (width 0.25) (layer F.Cu) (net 15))
 (segment (start 127.65 96.15) (end 127.65 97.85) (width 0.25) (layer F.Cu) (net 15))
 (segment (start 126.9 94.425) (end 126.9 95.4) (width 0.25) (layer F.Cu) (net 15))
 (segment (start 128.175001 111.654999) (end 127.849999 111.980001) (width 0.25) (layer F.Cu) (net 15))
 (segment (start 128.175001 101.825001) (end 128.175001 111.654999) (width 0.25) (layer F.Cu) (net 15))
 (segment (start 127.849999 111.980001) (end 127 112.83) (width 0.25) (layer F.Cu) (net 15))
 (segment (start 126.9 100.55) (end 128.175001 101.825001) (width 0.25) (layer F.Cu) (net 15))
 (segment (start 126.9 99.575) (end 126.9 100.55) (width 0.25) (layer F.Cu) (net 15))
 (segment (start 135.375001 101.975001) (end 135.3 101.9) (width 0.25) (layer F.Cu) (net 16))
 (segment (start 135.375001 108.035001) (end 135.375001 101.975001) (width 0.25) (layer F.Cu) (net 16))
 (segment (start 133.97499 122.17499) (end 133.97499 109.435012) (width 0.25) (layer F.Cu) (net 16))
 (segment (start 133.97499 109.435012) (end 135.375001 108.035001) (width 0.25) (layer F.Cu) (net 16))
 (segment (start 134.3 122.5) (end 133.97499 122.17499) (width 0.25) (layer F.Cu) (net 16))
 (segment (start 135.3 101.9) (end 134.3 101.9) (width 0.25) (layer F.Cu) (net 16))
 (segment (start 135 122.5) (end 134.3 122.5) (width 0.25) (layer F.Cu) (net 16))
 (segment (start 131.28681 101.1) (end 134.3 101.1) (width 0.25) (layer F.Cu) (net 17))
 (segment (start 130.72499 101.66182) (end 131.28681 101.1) (width 0.25) (layer F.Cu) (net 17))
 (segment (start 137.25 123.05) (end 136.89999 123.40001) (width 0.25) (layer F.Cu) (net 17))
 (segment (start 137.25 122.475) (end 137.25 123.05) (width 0.25) (layer F.Cu) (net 17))
 (segment (start 130.72499 119.81318) (end 130.72499 101.66182) (width 0.25) (layer F.Cu) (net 17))
 (segment (start 136.89999 123.40001) (end 134.31182 123.40001) (width 0.25) (layer F.Cu) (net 17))
 (segment (start 134.31182 123.40001) (end 130.72499 119.81318) (width 0.25) (layer F.Cu) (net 17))
 (segment (start 120.85 89.85) (end 121.825 89.85) (width 0.25) (layer B.Cu) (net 18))
 (segment (start 117.825001 89.674999) (end 120.674999 89.674999) (width 0.25) (layer B.Cu) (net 18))
 (segment (start 120.674999 89.674999) (end 120.85 89.85) (width 0.25) (layer B.Cu) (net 18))
 (segment (start 117.65 89.85) (end 117.825001 89.674999) (width 0.25) (layer B.Cu) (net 18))
 (segment (start 116.675 89.85) (end 117.65 89.85) (width 0.25) (layer B.Cu) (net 18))
 (segment (start 139.065685 107.5) (end 138.5 107.5) (width 0.25) (layer F.Cu) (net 18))
 (segment (start 140.1 107.5) (end 139.065685 107.5) (width 0.25) (layer F.Cu) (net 18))
 (segment (start 140.8 108.2) (end 140.1 107.5) (width 0.25) (layer F.Cu) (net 18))
 (segment (start 140.8 109.2) (end 140.8 108.2) (width 0.25) (layer F.Cu) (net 18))
 (segment (start 139.065685 107.5) (end 138.5 107.5) (width 0.25) (layer B.Cu) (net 18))
 (segment (start 142.225001 107.098001) (end 141.823002 107.5) (width 0.25) (layer B.Cu) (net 18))
 (segment (start 141.823002 107.5) (end 139.065685 107.5) (width 0.25) (layer B.Cu) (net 18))
 (segment (start 142.225001 106.102001) (end 142.225001 107.098001) (width 0.25) (layer B.Cu) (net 18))
 (segment (start 125.973 89.85) (end 142.225001 106.102001) (width 0.25) (layer B.Cu) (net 18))
 (segment (start 121.825 89.85) (end 125.973 89.85) (width 0.25) (layer B.Cu) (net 18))
 (segment (start 141.6 106.85) (end 141.5 106.75) (width 0.25) (layer F.Cu) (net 19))
 (segment (start 141.6 109.2) (end 141.6 106.85) (width 0.25) (layer F.Cu) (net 19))
 (segment (start 117.174999 112.075001) (end 117.35 111.9) (width 0.25) (layer B.Cu) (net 19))
 (segment (start 115.413999 112.075001) (end 117.174999 112.075001) (width 0.25) (layer B.Cu) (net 19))
 (segment (start 117.35 111.9) (end 118.325 111.9) (width 0.25) (layer B.Cu) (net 19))
 (segment (start 115.238998 111.9) (end 115.413999 112.075001) (width 0.25) (layer B.Cu) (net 19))
 (segment (start 113.175 111.9) (end 115.238998 111.9) (width 0.25) (layer B.Cu) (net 19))
 (segment (start 123.124999 106.350001) (end 141.100001 106.350001) (width 0.25) (layer B.Cu) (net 19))
 (segment (start 141.100001 106.350001) (end 141.5 106.75) (width 0.25) (layer B.Cu) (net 19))
 (segment (start 118.325 111.15) (end 123.124999 106.350001) (width 0.25) (layer B.Cu) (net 19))
 (segment (start 118.325 111.9) (end 118.325 111.15) (width 0.25) (layer B.Cu) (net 19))
 (segment (start 142.4 111.1) (end 142 111.5) (width 0.25) (layer F.Cu) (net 20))
 (segment (start 142.4 109.2) (end 142.4 111.1) (width 0.25) (layer F.Cu) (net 20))
 (segment (start 142 112.065685) (end 142 111.5) (width 0.25) (layer B.Cu) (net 20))
 (segment (start 150.95 121.65) (end 142 112.7) (width 0.25) (layer B.Cu) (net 20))
 (segment (start 142 112.7) (end 142 112.065685) (width 0.25) (layer B.Cu) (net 20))
 (segment (start 151.925 121.65) (end 150.95 121.65) (width 0.25) (layer B.Cu) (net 20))
 (segment (start 155.924999 121.825001) (end 156.1 121.65) (width 0.25) (layer B.Cu) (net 20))
 (segment (start 156.1 121.65) (end 157.075 121.65) (width 0.25) (layer B.Cu) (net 20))
 (segment (start 153.988998 121.65) (end 154.163999 121.825001) (width 0.25) (layer B.Cu) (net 20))
 (segment (start 154.163999 121.825001) (end 155.924999 121.825001) (width 0.25) (layer B.Cu) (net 20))
 (segment (start 151.925 121.65) (end 153.988998 121.65) (width 0.25) (layer B.Cu) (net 20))
 (segment (start 143.2 106.8) (end 143.25 106.75) (width 0.25) (layer F.Cu) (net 21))
 (segment (start 143.2 109.2) (end 143.2 106.8) (width 0.25) (layer F.Cu) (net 21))
 (segment (start 153.2 109.1) (end 153.425 109.1) (width 0.25) (layer B.Cu) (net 21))
 (segment (start 152.45 108.35) (end 153.2 109.1) (width 0.25) (layer B.Cu) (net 21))
 (segment (start 152.45 108.125) (end 152.45 108.35) (width 0.25) (layer B.Cu) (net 21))
 (segment (start 151.075 106.75) (end 152.45 108.125) (width 0.25) (layer B.Cu) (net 21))
 (segment (start 143.25 106.75) (end 151.075 106.75) (width 0.25) (layer B.Cu) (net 21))
 (segment (start 157.6 109.1) (end 158.575 109.1) (width 0.25) (layer B.Cu) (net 21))
 (segment (start 155.663999 108.924999) (end 157.424999 108.924999) (width 0.25) (layer B.Cu) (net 21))
 (segment (start 157.424999 108.924999) (end 157.6 109.1) (width 0.25) (layer B.Cu) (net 21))
 (segment (start 155.488998 109.1) (end 155.663999 108.924999) (width 0.25) (layer B.Cu) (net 21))
 (segment (start 153.425 109.1) (end 155.488998 109.1) (width 0.25) (layer B.Cu) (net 21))
 (segment (start 151.575001 91.674999) (end 151.4 91.85) (width 0.25) (layer B.Cu) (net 22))
 (segment (start 153.336001 91.674999) (end 151.575001 91.674999) (width 0.25) (layer B.Cu) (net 22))
 (segment (start 151.4 91.85) (end 150.425 91.85) (width 0.25) (layer B.Cu) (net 22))
 (segment (start 153.511002 91.85) (end 153.336001 91.674999) (width 0.25) (layer B.Cu) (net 22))
 (segment (start 155.575 91.85) (end 153.511002 91.85) (width 0.25) (layer B.Cu) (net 22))
 (segment (start 149.45 91.85) (end 147.5 93.8) (width 0.25) (layer B.Cu) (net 22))
 (segment (start 150.425 91.85) (end 149.45 91.85) (width 0.25) (layer B.Cu) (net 22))
 (segment (start 147.5 93.8) (end 147.5 105.024999) (width 0.25) (layer B.Cu) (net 22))
 (segment (start 147.5 105.024999) (end 147.5 105.75) (width 0.25) (layer B.Cu) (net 22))
 (segment (start 147.35 105.9) (end 147.5 105.75) (width 0.25) (layer F.Cu) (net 22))
 (segment (start 145.7 105.9) (end 147.35 105.9) (width 0.25) (layer F.Cu) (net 22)))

